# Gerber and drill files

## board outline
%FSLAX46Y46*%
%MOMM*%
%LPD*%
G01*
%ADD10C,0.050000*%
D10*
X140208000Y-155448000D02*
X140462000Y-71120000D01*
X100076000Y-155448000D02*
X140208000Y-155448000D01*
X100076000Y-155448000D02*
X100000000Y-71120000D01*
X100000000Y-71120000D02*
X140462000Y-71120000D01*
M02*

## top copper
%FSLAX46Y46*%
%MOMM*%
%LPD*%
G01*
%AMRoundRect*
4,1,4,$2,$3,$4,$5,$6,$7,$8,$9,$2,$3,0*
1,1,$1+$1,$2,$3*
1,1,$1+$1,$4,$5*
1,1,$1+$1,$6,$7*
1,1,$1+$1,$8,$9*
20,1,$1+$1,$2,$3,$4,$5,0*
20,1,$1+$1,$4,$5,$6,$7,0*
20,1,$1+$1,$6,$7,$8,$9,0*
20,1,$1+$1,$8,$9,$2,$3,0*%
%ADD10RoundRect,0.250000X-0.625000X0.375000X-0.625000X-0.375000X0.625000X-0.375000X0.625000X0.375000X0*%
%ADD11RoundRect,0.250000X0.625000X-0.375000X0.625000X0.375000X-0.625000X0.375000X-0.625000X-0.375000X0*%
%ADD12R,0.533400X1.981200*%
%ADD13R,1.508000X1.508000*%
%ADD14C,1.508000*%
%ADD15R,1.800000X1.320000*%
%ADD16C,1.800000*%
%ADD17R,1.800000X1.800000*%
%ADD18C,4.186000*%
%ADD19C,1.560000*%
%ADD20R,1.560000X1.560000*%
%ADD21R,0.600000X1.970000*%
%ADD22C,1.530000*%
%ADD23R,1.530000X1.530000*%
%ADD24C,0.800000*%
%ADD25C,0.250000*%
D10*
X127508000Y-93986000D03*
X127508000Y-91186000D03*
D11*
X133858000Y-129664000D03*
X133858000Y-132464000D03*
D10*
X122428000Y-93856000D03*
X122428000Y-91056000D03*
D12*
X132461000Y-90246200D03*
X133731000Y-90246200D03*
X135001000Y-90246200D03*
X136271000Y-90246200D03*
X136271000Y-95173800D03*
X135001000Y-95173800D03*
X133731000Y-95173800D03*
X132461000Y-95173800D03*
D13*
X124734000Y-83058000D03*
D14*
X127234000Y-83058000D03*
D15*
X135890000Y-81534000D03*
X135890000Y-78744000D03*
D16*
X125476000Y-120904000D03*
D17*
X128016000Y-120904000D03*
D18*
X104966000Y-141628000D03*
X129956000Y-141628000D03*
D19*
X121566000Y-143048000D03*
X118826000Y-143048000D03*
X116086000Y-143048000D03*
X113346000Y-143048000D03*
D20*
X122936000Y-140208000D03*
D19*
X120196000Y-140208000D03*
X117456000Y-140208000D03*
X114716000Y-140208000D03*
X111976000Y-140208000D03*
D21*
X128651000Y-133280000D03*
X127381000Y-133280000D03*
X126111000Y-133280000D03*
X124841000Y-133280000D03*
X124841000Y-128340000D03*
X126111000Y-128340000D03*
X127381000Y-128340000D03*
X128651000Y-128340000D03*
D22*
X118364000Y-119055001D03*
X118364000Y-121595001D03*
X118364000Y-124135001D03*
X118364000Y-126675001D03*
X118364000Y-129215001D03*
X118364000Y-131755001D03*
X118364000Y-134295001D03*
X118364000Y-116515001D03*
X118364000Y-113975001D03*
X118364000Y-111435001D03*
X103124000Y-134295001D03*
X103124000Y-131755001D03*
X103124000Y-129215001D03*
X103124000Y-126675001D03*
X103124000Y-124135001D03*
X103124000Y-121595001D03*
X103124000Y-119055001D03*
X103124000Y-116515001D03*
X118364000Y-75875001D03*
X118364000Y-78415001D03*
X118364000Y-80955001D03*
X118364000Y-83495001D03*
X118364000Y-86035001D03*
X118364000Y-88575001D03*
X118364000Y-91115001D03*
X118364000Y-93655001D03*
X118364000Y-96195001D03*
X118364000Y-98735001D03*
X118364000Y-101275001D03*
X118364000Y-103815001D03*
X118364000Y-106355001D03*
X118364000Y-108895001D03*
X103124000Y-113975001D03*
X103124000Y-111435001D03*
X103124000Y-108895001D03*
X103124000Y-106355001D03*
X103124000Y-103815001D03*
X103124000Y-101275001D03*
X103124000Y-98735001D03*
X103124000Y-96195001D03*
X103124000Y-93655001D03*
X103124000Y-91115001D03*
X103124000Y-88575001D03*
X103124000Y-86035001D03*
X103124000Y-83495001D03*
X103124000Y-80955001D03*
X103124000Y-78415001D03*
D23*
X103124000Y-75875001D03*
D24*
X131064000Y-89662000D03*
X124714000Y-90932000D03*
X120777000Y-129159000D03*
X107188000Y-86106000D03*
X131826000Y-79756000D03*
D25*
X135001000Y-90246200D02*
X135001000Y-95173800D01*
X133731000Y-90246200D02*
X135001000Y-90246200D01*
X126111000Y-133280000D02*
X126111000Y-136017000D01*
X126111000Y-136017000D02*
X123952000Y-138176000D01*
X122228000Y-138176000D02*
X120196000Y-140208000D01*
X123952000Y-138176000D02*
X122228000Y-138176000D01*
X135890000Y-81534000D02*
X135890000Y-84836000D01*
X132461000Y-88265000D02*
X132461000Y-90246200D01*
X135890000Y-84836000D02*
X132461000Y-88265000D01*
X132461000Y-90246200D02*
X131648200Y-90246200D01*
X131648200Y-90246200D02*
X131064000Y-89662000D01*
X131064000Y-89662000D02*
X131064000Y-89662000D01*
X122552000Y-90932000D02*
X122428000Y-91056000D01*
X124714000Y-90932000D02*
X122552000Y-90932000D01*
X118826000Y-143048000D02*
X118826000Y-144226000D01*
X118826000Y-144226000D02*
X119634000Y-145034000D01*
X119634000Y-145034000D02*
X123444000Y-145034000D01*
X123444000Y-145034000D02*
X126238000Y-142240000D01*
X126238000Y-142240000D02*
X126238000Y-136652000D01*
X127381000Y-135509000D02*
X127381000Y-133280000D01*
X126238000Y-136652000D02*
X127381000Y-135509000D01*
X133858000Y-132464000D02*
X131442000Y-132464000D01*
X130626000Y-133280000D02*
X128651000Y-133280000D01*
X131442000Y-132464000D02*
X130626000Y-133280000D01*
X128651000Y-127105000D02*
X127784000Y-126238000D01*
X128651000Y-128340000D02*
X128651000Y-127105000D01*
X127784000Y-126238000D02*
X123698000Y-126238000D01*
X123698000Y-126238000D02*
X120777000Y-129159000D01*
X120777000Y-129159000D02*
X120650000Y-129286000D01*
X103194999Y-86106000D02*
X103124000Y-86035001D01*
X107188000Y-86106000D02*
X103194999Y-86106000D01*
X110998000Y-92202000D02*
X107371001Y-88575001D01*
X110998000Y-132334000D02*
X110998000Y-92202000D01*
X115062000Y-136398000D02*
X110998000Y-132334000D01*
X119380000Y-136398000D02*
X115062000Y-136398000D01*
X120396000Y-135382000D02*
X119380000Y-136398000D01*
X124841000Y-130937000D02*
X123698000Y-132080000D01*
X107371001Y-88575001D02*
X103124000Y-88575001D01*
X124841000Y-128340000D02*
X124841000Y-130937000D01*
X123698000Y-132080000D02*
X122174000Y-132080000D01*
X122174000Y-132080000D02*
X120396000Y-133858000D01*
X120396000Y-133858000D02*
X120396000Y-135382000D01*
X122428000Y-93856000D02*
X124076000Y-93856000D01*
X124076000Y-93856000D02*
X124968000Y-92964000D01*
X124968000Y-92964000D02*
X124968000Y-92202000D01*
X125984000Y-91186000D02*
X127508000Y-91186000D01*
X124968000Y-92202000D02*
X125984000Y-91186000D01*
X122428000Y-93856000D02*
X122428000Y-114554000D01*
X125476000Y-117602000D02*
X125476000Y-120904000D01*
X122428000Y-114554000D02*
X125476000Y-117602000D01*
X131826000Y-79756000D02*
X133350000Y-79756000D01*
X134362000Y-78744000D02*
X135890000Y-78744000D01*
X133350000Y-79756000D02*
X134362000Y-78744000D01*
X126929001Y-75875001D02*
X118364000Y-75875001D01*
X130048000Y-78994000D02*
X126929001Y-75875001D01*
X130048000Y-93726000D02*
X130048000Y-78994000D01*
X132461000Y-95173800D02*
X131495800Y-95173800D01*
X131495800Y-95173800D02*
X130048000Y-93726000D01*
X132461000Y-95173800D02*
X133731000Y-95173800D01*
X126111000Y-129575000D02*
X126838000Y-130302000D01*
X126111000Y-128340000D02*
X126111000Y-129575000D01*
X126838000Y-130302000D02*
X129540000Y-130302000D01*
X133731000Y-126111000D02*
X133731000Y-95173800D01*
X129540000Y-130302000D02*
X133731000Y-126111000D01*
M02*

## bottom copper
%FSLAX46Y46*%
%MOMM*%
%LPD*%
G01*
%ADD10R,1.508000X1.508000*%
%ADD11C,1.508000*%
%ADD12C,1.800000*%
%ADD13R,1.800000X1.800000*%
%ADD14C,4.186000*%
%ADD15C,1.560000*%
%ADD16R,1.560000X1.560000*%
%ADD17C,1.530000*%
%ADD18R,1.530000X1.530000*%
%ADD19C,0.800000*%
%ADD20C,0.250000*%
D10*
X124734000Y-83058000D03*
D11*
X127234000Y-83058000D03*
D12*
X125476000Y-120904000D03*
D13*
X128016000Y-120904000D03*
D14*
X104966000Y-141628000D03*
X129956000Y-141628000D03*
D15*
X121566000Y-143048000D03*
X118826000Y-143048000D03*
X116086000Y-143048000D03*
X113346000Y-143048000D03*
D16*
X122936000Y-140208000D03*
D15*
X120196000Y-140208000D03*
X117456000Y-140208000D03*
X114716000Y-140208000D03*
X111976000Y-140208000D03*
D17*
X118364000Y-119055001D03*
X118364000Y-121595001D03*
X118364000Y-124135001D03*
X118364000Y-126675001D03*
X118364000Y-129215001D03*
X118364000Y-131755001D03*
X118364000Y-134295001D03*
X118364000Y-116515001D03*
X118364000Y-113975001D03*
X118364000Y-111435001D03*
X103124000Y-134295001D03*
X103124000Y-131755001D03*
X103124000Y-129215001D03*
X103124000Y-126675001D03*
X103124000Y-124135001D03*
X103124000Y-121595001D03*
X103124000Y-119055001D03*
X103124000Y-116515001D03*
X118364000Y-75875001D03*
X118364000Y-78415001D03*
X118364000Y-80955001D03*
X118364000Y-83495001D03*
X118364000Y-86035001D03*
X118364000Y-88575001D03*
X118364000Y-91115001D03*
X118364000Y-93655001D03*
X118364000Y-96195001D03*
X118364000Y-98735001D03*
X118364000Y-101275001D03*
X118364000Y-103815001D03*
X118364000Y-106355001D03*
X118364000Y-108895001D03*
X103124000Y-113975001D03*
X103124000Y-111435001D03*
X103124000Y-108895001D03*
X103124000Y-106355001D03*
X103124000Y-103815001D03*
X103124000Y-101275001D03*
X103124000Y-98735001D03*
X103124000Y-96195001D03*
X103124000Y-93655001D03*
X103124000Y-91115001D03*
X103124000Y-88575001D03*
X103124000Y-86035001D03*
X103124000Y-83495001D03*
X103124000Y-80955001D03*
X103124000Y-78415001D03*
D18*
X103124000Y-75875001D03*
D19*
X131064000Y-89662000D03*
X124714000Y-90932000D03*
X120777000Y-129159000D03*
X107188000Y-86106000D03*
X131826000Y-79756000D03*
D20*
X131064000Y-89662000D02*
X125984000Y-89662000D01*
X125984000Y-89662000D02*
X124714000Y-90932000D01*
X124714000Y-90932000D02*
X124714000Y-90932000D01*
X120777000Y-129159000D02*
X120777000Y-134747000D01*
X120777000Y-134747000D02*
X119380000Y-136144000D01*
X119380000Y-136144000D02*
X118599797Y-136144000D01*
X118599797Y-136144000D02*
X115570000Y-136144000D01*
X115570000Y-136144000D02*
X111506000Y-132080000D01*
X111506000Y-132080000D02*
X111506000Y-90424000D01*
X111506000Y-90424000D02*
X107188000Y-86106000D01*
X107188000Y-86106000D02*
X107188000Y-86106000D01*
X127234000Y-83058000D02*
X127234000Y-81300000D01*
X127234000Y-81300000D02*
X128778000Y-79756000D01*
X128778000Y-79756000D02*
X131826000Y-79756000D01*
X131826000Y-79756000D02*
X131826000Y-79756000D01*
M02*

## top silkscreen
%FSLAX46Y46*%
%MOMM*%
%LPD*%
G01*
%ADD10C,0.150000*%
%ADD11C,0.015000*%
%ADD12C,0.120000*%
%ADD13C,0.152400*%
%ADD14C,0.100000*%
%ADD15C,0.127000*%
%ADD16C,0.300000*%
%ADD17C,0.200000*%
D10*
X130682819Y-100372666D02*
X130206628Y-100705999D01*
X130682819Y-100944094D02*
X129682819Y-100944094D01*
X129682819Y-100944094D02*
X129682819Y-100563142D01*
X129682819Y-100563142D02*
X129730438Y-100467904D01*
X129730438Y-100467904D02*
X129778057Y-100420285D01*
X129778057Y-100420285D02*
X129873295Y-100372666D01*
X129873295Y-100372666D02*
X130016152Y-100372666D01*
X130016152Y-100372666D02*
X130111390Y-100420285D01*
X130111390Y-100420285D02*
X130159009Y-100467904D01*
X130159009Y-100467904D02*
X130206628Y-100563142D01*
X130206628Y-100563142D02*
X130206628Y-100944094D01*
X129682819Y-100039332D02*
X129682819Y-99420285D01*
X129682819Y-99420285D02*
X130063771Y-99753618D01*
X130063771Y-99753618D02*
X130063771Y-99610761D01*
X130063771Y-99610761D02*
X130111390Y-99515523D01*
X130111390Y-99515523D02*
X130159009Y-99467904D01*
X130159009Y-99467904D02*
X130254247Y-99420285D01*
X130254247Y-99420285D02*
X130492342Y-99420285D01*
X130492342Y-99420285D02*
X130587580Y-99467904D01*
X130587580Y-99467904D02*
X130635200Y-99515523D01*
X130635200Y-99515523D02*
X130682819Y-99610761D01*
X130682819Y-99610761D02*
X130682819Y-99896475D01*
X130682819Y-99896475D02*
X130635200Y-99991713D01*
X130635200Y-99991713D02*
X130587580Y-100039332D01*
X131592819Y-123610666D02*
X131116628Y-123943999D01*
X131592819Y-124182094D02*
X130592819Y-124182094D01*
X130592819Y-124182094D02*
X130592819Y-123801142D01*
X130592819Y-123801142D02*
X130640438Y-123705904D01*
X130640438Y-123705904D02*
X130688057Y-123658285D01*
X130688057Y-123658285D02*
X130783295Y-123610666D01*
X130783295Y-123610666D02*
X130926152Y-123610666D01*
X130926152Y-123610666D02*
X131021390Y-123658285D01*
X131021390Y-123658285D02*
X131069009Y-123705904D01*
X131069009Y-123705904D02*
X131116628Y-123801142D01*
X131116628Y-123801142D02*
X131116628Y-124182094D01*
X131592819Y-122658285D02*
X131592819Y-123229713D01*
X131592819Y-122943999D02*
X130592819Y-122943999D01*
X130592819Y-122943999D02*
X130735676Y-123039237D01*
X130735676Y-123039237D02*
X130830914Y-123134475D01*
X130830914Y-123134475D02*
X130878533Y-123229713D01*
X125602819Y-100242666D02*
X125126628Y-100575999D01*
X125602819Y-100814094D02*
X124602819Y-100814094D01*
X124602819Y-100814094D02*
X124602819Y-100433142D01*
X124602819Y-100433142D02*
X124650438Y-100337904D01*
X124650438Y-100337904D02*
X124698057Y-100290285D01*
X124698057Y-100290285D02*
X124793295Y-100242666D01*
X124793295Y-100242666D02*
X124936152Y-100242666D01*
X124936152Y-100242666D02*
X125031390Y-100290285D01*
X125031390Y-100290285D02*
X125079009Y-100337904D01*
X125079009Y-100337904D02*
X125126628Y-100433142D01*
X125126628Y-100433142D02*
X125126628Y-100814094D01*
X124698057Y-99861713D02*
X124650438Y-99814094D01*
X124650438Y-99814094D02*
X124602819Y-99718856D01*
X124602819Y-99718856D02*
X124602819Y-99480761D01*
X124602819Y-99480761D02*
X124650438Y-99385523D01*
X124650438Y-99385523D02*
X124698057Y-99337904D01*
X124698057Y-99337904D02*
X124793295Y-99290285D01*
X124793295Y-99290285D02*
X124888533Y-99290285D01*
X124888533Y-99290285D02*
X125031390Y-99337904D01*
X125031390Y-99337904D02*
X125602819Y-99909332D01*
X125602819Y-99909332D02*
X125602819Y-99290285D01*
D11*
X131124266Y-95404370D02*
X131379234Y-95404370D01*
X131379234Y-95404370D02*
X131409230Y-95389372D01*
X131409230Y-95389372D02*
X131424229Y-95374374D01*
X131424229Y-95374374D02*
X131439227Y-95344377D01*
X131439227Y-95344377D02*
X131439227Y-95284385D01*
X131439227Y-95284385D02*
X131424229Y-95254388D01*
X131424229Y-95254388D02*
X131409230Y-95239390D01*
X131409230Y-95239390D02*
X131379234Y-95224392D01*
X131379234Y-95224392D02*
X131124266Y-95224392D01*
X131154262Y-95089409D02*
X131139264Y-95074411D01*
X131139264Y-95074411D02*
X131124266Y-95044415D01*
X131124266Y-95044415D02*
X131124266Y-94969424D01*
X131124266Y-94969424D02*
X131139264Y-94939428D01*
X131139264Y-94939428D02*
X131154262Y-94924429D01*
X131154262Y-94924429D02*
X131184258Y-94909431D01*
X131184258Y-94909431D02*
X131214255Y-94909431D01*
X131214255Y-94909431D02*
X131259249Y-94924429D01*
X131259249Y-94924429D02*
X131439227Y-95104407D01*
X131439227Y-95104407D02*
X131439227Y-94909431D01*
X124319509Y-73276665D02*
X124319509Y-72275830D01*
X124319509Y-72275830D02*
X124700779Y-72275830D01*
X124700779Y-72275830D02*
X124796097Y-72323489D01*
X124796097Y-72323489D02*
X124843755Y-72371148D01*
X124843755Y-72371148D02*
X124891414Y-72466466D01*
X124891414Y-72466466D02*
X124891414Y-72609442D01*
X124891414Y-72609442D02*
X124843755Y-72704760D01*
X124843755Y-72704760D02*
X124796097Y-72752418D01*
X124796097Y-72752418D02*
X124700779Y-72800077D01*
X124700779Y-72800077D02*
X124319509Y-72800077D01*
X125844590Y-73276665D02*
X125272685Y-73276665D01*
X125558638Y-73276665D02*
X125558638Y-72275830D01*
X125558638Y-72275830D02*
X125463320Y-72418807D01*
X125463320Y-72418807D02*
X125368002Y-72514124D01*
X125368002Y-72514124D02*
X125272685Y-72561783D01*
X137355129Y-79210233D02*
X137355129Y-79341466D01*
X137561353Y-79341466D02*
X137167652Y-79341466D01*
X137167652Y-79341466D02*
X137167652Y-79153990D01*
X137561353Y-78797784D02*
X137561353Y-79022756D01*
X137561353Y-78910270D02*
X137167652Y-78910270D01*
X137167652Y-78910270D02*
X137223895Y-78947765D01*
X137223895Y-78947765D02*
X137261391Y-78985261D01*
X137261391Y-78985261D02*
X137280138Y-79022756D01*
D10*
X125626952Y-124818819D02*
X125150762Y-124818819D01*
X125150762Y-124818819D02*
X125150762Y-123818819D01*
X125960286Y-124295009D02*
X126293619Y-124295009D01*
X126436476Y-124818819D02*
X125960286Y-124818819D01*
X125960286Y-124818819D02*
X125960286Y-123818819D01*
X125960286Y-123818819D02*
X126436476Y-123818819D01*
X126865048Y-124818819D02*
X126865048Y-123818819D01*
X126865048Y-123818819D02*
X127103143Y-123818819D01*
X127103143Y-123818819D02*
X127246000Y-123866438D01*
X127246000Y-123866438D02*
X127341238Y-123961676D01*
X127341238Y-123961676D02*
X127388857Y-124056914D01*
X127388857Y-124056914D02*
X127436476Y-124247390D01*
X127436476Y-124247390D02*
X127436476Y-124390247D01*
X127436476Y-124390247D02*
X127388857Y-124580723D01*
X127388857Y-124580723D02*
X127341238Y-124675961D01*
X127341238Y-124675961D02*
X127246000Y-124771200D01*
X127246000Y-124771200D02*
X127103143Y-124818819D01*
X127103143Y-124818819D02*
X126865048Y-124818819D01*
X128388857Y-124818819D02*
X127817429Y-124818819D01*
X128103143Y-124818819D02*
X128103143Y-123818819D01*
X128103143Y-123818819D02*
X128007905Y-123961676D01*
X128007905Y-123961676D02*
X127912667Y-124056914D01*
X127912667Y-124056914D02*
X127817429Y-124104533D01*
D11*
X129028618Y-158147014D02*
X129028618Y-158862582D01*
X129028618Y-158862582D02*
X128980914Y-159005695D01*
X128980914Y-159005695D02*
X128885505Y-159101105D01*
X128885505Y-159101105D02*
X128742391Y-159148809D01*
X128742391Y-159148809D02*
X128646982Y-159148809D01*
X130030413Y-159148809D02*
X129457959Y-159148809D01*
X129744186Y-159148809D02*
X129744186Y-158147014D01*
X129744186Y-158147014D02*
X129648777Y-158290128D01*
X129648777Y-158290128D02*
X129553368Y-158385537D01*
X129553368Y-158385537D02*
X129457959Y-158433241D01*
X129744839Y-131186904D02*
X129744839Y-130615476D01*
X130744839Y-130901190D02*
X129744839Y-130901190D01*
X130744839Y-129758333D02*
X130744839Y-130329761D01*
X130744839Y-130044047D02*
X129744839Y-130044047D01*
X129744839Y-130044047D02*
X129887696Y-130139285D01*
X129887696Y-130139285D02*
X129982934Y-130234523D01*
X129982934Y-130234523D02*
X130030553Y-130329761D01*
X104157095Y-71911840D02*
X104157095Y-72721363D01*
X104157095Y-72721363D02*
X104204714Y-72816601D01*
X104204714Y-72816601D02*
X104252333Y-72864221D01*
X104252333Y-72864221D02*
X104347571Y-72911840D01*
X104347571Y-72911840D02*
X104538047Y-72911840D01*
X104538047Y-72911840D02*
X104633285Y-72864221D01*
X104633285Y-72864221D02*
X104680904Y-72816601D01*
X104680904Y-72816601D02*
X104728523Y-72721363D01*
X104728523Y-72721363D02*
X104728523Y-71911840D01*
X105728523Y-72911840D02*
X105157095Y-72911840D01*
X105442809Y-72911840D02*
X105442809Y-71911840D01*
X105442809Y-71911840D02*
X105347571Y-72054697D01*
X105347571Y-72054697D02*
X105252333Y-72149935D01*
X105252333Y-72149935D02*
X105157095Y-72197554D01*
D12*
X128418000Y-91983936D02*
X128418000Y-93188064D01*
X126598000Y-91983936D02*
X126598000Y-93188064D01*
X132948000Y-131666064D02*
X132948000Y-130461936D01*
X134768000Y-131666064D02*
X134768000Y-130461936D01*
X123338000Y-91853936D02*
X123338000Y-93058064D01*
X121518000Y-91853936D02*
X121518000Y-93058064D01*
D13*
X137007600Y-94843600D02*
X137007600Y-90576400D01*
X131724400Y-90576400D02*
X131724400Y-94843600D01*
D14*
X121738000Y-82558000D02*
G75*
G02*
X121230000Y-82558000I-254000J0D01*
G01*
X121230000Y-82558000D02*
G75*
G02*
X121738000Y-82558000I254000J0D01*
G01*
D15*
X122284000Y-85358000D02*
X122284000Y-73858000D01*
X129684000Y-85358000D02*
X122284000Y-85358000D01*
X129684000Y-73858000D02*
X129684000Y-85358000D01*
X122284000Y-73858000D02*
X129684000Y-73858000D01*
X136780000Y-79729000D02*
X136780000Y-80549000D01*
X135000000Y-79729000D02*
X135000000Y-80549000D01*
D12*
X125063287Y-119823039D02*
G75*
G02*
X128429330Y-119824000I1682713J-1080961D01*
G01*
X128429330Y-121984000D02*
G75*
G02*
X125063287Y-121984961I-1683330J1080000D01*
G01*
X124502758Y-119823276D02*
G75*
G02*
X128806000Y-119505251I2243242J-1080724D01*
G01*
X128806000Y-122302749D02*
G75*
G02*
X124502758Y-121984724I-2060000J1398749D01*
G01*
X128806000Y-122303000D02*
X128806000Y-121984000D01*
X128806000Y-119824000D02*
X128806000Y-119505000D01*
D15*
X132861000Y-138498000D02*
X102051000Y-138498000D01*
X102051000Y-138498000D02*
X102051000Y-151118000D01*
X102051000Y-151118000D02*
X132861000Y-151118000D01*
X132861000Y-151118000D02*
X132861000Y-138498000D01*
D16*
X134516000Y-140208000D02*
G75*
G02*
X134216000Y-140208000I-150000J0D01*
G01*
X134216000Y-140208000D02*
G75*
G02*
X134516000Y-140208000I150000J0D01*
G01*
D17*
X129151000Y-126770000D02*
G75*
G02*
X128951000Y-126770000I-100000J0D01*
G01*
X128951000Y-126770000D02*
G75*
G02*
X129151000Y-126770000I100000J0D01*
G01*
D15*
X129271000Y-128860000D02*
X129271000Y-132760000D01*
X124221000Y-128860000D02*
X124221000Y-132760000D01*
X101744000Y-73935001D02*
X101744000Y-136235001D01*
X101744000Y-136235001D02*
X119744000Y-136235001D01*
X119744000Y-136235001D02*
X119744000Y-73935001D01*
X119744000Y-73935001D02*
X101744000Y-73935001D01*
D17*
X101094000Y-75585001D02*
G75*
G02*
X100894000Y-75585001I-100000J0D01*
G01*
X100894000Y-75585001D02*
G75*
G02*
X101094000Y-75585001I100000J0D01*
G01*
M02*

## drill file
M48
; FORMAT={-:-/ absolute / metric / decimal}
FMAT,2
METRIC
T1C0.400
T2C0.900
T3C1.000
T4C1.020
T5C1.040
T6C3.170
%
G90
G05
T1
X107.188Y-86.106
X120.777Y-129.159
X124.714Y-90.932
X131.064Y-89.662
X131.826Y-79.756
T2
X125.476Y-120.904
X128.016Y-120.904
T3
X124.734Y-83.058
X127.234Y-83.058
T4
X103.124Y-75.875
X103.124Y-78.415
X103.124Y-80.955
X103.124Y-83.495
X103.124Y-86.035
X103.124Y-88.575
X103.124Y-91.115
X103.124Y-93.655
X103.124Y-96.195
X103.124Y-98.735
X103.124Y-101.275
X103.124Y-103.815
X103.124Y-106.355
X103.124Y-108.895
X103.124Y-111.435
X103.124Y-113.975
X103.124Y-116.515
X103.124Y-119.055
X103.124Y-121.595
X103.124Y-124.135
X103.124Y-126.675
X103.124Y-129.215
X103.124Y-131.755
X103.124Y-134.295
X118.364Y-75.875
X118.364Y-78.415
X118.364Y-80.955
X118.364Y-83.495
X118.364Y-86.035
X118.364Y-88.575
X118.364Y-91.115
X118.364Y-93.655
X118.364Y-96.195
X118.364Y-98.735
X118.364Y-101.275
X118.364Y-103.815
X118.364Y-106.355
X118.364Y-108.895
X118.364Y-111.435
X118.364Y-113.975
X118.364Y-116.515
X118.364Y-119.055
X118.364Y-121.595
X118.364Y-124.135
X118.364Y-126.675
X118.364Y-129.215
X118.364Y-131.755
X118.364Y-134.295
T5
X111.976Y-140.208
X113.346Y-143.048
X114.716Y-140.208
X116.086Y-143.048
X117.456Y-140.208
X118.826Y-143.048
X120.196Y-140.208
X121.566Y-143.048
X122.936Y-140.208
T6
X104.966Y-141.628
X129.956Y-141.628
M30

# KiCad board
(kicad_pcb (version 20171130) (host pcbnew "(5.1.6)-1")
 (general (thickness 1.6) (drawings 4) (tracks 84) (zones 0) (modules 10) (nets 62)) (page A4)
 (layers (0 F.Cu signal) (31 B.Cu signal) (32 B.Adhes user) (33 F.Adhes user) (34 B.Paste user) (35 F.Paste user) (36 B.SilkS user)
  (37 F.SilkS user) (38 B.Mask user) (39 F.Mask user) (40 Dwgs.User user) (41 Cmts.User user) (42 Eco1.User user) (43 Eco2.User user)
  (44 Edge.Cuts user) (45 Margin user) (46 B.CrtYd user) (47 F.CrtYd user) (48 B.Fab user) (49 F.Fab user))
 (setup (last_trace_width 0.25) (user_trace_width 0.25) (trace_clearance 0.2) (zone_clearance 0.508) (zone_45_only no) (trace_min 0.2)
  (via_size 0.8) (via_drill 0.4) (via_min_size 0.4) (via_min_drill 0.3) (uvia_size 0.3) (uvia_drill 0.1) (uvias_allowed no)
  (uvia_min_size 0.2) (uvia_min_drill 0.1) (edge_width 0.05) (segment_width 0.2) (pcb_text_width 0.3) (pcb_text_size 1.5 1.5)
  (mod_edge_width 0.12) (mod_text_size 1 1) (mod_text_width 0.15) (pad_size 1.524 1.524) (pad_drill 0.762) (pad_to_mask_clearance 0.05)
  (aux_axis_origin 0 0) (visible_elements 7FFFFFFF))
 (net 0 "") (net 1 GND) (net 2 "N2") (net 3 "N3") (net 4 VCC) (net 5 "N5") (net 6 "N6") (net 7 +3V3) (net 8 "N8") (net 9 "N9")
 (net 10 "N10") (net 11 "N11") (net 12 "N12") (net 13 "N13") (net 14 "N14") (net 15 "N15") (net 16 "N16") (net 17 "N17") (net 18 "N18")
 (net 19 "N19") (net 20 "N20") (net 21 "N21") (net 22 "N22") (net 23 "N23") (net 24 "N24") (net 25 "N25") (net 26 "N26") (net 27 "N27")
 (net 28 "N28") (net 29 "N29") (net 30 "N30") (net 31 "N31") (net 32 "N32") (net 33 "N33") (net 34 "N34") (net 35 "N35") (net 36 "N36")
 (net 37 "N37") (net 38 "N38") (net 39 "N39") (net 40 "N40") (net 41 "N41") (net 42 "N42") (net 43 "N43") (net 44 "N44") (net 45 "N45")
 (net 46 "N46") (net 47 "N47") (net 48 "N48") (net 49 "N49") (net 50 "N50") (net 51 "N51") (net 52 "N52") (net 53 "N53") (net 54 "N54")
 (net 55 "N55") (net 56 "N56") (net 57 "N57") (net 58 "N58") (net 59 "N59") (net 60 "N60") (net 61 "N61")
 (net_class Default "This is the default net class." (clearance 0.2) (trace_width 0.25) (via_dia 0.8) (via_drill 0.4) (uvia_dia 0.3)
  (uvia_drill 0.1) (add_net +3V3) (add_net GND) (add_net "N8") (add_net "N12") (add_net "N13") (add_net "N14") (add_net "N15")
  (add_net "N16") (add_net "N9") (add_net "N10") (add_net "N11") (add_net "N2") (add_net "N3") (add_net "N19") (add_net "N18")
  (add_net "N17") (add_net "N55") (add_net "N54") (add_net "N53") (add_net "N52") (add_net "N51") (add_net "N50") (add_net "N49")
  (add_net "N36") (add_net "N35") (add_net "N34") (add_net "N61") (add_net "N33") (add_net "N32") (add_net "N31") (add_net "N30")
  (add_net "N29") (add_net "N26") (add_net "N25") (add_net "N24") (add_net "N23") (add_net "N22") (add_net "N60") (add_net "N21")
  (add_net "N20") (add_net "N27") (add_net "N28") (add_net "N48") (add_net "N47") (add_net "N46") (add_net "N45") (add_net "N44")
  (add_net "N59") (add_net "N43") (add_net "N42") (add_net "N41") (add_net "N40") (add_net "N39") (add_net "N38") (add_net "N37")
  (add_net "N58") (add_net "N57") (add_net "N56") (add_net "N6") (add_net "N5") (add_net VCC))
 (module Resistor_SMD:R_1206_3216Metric (layer F.Cu) (at 127.508 92.586 270)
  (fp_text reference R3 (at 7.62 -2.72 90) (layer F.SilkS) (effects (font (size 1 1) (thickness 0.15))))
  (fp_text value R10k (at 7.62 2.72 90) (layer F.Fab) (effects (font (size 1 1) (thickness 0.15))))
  (fp_line (start -0.602064 -0.91) (end 0.602064 -0.91) (layer F.SilkS) (width 0.12))
  (fp_line (start -0.602064 0.91) (end 0.602064 0.91) (layer F.SilkS) (width 0.12))
  (pad 2 smd roundrect (at 1.4 0 270) (size 1.25 1.75) (layers F.Cu F.Paste F.Mask) (roundrect_rratio 0.2) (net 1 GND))
  (pad 1 smd roundrect (at -1.4 0 270) (size 1.25 1.75) (layers F.Cu F.Paste F.Mask) (roundrect_rratio 0.2) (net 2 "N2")))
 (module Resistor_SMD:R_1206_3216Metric (layer F.Cu) (at 133.858 131.064 90)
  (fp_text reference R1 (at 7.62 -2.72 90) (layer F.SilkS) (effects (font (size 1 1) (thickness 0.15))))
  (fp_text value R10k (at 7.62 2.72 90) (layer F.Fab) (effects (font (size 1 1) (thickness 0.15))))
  (fp_line (start -0.602064 -0.91) (end 0.602064 -0.91) (layer F.SilkS) (width 0.12))
  (fp_line (start -0.602064 0.91) (end 0.602064 0.91) (layer F.SilkS) (width 0.12))
  (pad 2 smd roundrect (at 1.4 0 90) (size 1.25 1.75) (layers F.Cu F.Paste F.Mask) (roundrect_rratio 0.2) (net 1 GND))
  (pad 1 smd roundrect (at -1.4 0 90) (size 1.25 1.75) (layers F.Cu F.Paste F.Mask) (roundrect_rratio 0.2) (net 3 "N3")))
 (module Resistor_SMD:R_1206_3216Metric (layer F.Cu) (at 122.428 92.456 270)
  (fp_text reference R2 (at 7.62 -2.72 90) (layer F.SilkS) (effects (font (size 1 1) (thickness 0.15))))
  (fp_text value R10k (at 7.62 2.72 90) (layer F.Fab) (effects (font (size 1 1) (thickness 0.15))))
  (fp_line (start -0.602064 -0.91) (end 0.602064 -0.91) (layer F.SilkS) (width 0.12))
  (fp_line (start -0.602064 0.91) (end 0.602064 0.91) (layer F.SilkS) (width 0.12))
  (pad 2 smd roundrect (at 1.4 0 270) (size 1.25 1.75) (layers F.Cu F.Paste F.Mask) (roundrect_rratio 0.2) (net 2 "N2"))
  (pad 1 smd roundrect (at -1.4 0 270) (size 1.25 1.75) (layers F.Cu F.Paste F.Mask) (roundrect_rratio 0.2) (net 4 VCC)))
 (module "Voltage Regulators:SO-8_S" (layer F.Cu) (at 134.366 92.71 90)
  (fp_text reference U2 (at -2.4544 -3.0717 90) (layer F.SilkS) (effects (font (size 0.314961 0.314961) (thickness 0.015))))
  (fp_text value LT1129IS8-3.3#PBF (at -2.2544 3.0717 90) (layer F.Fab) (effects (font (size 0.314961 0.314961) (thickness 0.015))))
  (fp_line (start -2.1336 2.6416) (end 2.1336 2.6416) (layer F.SilkS) (width 0.1524))
  (fp_line (start 2.1336 -2.6416) (end -2.1336 -2.6416) (layer F.SilkS) (width 0.1524))
  (pad 8 smd rect (at 2.4638 -1.905 90) (size 1.9812 0.5334) (layers F.Cu F.Paste F.Mask) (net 4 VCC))
  (pad 7 smd rect (at 2.4638 -0.635 90) (size 1.9812 0.5334) (layers F.Cu F.Paste F.Mask) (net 1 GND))
  (pad 6 smd rect (at 2.4638 0.635 90) (size 1.9812 0.5334) (layers F.Cu F.Paste F.Mask) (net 1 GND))
  (pad 5 smd rect (at 2.4638 1.905 90) (size 1.9812 0.5334) (layers F.Cu F.Paste F.Mask) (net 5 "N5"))
  (pad 4 smd rect (at -2.4638 1.905 90) (size 1.9812 0.5334) (layers F.Cu F.Paste F.Mask) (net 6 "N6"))
  (pad 3 smd rect (at -2.4638 0.635 90) (size 1.9812 0.5334) (layers F.Cu F.Paste F.Mask) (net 1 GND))
  (pad 2 smd rect (at -2.4638 -0.635 90) (size 1.9812 0.5334) (layers F.Cu F.Paste F.Mask) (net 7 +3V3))
  (pad 1 smd rect (at -2.4638 -1.905 90) (size 1.9812 0.5334) (layers F.Cu F.Paste F.Mask) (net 7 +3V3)))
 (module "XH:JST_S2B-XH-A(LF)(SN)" (layer F.Cu) (at 125.984 83.058)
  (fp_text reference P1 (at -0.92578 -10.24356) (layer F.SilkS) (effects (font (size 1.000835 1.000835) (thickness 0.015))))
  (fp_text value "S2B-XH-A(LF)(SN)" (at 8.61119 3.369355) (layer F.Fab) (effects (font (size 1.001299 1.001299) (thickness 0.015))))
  (fp_circle (center -4.5 -0.5) (end -4.246 -0.5) (layer F.SilkS) (width 0.1))
  (fp_line (start -3.7 2.3) (end -3.7 -9.2) (layer F.SilkS) (width 0.127))
  (fp_line (start 3.7 2.3) (end -3.7 2.3) (layer F.SilkS) (width 0.127))
  (fp_line (start 3.7 -9.2) (end 3.7 2.3) (layer F.SilkS) (width 0.127))
  (fp_line (start -3.7 -9.2) (end 3.7 -9.2) (layer F.SilkS) (width 0.127))
  (pad 1 thru_hole rect (at -1.25 0) (size 1.508 1.508) (drill 1) (layers *.Cu *.Mask) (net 1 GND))
  (pad 2 thru_hole circle (at 1.25 0) (size 1.508 1.508) (drill 1) (layers *.Cu *.Mask) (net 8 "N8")))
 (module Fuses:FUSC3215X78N (layer F.Cu) (at 135.89 80.139 270)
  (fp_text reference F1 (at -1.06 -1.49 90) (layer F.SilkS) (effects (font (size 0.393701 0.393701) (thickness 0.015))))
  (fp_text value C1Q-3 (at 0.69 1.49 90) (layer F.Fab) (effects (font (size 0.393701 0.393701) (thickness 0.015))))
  (fp_line (start -0.41 -0.89) (end 0.41 -0.89) (layer F.SilkS) (width 0.127))
  (fp_line (start -0.41 0.89) (end 0.41 0.89) (layer F.SilkS) (width 0.127))
  (pad 2 smd rect (at 1.395 0 270) (size 1.32 1.8) (layers F.Cu F.Paste F.Mask) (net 4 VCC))
  (pad 1 smd rect (at -1.395 0 270) (size 1.32 1.8) (layers F.Cu F.Paste F.Mask) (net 8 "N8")))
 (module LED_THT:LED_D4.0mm (layer F.Cu) (at 128.016 120.904 180)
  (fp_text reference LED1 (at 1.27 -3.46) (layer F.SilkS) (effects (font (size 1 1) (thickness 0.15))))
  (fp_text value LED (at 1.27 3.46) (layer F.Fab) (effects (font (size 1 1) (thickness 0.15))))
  (fp_arc (start 1.27 0) (end -0.41333 1.08) (angle -114.6) (layer F.SilkS) (width 0.12))
  (fp_arc (start 1.27 0) (end -0.41333 -1.08) (angle 114.6) (layer F.SilkS) (width 0.12))
  (fp_arc (start 1.27 0) (end -0.79 1.398749) (angle -120.1) (layer F.SilkS) (width 0.12))
  (fp_arc (start 1.27 0) (end -0.79 -1.398749) (angle 120.1) (layer F.SilkS) (width 0.12))
  (fp_line (start -0.79 -1.399) (end -0.79 -1.08) (layer F.SilkS) (width 0.12))
  (fp_line (start -0.79 1.08) (end -0.79 1.399) (layer F.SilkS) (width 0.12))
  (pad 2 thru_hole circle (at 2.54 0 180) (size 1.8 1.8) (drill 0.9) (layers *.Cu *.Mask) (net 2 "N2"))
  (pad 1 thru_hole rect (at 0 0 180) (size 1.8 1.8) (drill 0.9) (layers *.Cu *.Mask) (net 1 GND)))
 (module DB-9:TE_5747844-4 (layer F.Cu) (at 122.936 140.208 180)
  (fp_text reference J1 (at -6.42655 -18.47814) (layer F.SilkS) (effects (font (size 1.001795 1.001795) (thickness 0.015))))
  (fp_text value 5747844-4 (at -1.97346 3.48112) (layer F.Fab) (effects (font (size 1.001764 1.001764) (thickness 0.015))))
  (fp_line (start -9.925 1.71) (end 20.885 1.71) (layer F.SilkS) (width 0.127))
  (fp_line (start 20.885 1.71) (end 20.885 -10.91) (layer F.SilkS) (width 0.127))
  (fp_line (start 20.885 -10.91) (end -9.925 -10.91) (layer F.SilkS) (width 0.127))
  (fp_line (start -9.925 -10.91) (end -9.925 1.71) (layer F.SilkS) (width 0.127))
  (fp_circle (center -11.43 0) (end -11.28 0) (layer F.SilkS) (width 0.3))
  (pad SH2 thru_hole circle (at 17.97 -1.42 180) (size 4.186 4.186) (drill 3.17) (layers *.Cu *.Mask) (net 1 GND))
  (pad SH1 thru_hole circle (at -7.02 -1.42 180) (size 4.186 4.186) (drill 3.17) (layers *.Cu *.Mask) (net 1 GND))
  (pad 6 thru_hole circle (at 1.37 -2.84 180) (size 1.56 1.56) (drill 1.04) (layers *.Cu *.Mask) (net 1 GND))
  (pad 7 thru_hole circle (at 4.11 -2.84 180) (size 1.56 1.56) (drill 1.04) (layers *.Cu *.Mask) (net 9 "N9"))
  (pad 8 thru_hole circle (at 6.85 -2.84 180) (size 1.56 1.56) (drill 1.04) (layers *.Cu *.Mask) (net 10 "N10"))
  (pad 9 thru_hole circle (at 9.59 -2.84 180) (size 1.56 1.56) (drill 1.04) (layers *.Cu *.Mask) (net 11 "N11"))
  (pad 1 thru_hole rect (at 0 0 180) (size 1.56 1.56) (drill 1.04) (layers *.Cu *.Mask) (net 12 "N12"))
  (pad 2 thru_hole circle (at 2.74 0 180) (size 1.56 1.56) (drill 1.04) (layers *.Cu *.Mask) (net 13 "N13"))
  (pad 3 thru_hole circle (at 5.48 0 180) (size 1.56 1.56) (drill 1.04) (layers *.Cu *.Mask) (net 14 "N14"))
  (pad 4 thru_hole circle (at 8.22 0 180) (size 1.56 1.56) (drill 1.04) (layers *.Cu *.Mask) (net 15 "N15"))
  (pad 5 thru_hole circle (at 10.96 0 180) (size 1.56 1.56) (drill 1.04) (layers *.Cu *.Mask) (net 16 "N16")))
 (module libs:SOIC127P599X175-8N (layer F.Cu) (at 126.746 130.81 270)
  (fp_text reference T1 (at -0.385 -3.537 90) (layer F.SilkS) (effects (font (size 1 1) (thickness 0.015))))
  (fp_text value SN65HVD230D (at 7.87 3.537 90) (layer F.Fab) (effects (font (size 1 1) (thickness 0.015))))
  (fp_circle (center -4.04 -2.305) (end -3.94 -2.305) (layer F.SilkS) (width 0.2))
  (fp_line (start -1.95 -2.525) (end 1.95 -2.525) (layer F.SilkS) (width 0.127))
  (fp_line (start -1.95 2.525) (end 1.95 2.525) (layer F.SilkS) (width 0.127))
  (pad 8 smd rect (at 2.47 -1.905 270) (size 1.97 0.6) (layers F.Cu F.Paste F.Mask) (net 3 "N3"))
  (pad 7 smd rect (at 2.47 -0.635 270) (size 1.97 0.6) (layers F.Cu F.Paste F.Mask) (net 9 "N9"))
  (pad 6 smd rect (at 2.47 0.635 270) (size 1.97 0.6) (layers F.Cu F.Paste F.Mask) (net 13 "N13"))
  (pad 5 smd rect (at 2.47 1.905 270) (size 1.97 0.6) (layers F.Cu F.Paste F.Mask) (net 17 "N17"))
  (pad 4 smd rect (at -2.47 1.905 270) (size 1.97 0.6) (layers F.Cu F.Paste F.Mask) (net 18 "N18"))
  (pad 3 smd rect (at -2.47 0.635 270) (size 1.97 0.6) (layers F.Cu F.Paste F.Mask) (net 7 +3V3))
  (pad 2 smd rect (at -2.47 -0.635 270) (size 1.97 0.6) (layers F.Cu F.Paste F.Mask) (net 1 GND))
  (pad 1 smd rect (at -2.47 -1.905 270) (size 1.97 0.6) (layers F.Cu F.Paste F.Mask) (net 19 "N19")))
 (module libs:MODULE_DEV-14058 (layer F.Cu) (at 110.744 105.085001)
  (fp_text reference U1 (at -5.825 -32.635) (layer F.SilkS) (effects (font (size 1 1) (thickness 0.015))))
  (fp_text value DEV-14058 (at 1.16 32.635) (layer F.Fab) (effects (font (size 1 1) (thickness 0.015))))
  (fp_line (start -9 -31.15) (end -9 31.15) (layer F.SilkS) (width 0.127))
  (fp_line (start -9 31.15) (end 9 31.15) (layer F.SilkS) (width 0.127))
  (fp_line (start 9 31.15) (end 9 -31.15) (layer F.SilkS) (width 0.127))
  (fp_line (start 9 -31.15) (end -9 -31.15) (layer F.SilkS) (width 0.127))
  (fp_circle (center -9.75 -29.5) (end -9.65 -29.5) (layer F.SilkS) (width 0.2))
  (pad 31 thru_hole circle (at 7.62 13.97) (size 1.53 1.53) (drill 1.02) (layers *.Cu *.Mask) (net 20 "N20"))
  (pad 30 thru_hole circle (at 7.62 16.51) (size 1.53 1.53) (drill 1.02) (layers *.Cu *.Mask) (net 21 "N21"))
  (pad 29 thru_hole circle (at 7.62 19.05) (size 1.53 1.53) (drill 1.02) (layers *.Cu *.Mask) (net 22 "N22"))
  (pad 28 thru_hole circle (at 7.62 21.59) (size 1.53 1.53) (drill 1.02) (layers *.Cu *.Mask) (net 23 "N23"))
  (pad 27 thru_hole circle (at 7.62 24.13) (size 1.53 1.53) (drill 1.02) (layers *.Cu *.Mask) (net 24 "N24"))
  (pad 26 thru_hole circle (at 7.62 26.67) (size 1.53 1.53) (drill 1.02) (layers *.Cu *.Mask) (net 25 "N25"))
  (pad 25 thru_hole circle (at 7.62 29.21) (size 1.53 1.53) (drill 1.02) (layers *.Cu *.Mask) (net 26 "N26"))
  (pad 32 thru_hole circle (at 7.62 11.43) (size 1.53 1.53) (drill 1.02) (layers *.Cu *.Mask) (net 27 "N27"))
  (pad 33 thru_hole circle (at 7.62 8.89) (size 1.53 1.53) (drill 1.02) (layers *.Cu *.Mask) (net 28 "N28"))
  (pad 34 thru_hole circle (at 7.62 6.35) (size 1.53 1.53) (drill 1.02) (layers *.Cu *.Mask) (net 1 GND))
  (pad 24 thru_hole circle (at -7.62 29.21) (size 1.53 1.53) (drill 1.02) (layers *.Cu *.Mask) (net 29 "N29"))
  (pad 23 thru_hole circle (at -7.62 26.67) (size 1.53 1.53) (drill 1.02) (layers *.Cu *.Mask) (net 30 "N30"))
  (pad 22 thru_hole circle (at -7.62 24.13) (size 1.53 1.53) (drill 1.02) (layers *.Cu *.Mask) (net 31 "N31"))
  (pad 21 thru_hole circle (at -7.62 21.59) (size 1.53 1.53) (drill 1.02) (layers *.Cu *.Mask) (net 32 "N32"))
  (pad 20 thru_hole circle (at -7.62 19.05) (size 1.53 1.53) (drill 1.02) (layers *.Cu *.Mask) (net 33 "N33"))
  (pad 19 thru_hole circle (at -7.62 16.51) (size 1.53 1.53) (drill 1.02) (layers *.Cu *.Mask) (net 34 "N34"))
  (pad 18 thru_hole circle (at -7.62 13.97) (size 1.53 1.53) (drill 1.02) (layers *.Cu *.Mask) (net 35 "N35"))
  (pad 17 thru_hole circle (at -7.62 11.43) (size 1.53 1.53) (drill 1.02) (layers *.Cu *.Mask) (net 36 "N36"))
  (pad 48 thru_hole circle (at 7.62 -29.21) (size 1.53 1.53) (drill 1.02) (layers *.Cu *.Mask) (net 7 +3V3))
  (pad 47 thru_hole circle (at 7.62 -26.67) (size 1.53 1.53) (drill 1.02) (layers *.Cu *.Mask) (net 1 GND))
  (pad 46 thru_hole circle (at 7.62 -24.13) (size 1.53 1.53) (drill 1.02) (layers *.Cu *.Mask) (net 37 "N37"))
  (pad 45 thru_hole circle (at 7.62 -21.59) (size 1.53 1.53) (drill 1.02) (layers *.Cu *.Mask) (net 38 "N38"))
  (pad 44 thru_hole circle (at 7.62 -19.05) (size 1.53 1.53) (drill 1.02) (layers *.Cu *.Mask) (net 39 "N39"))
  (pad 43 thru_hole circle (at 7.62 -16.51) (size 1.53 1.53) (drill 1.02) (layers *.Cu *.Mask) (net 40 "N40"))
  (pad 42 thru_hole circle (at 7.62 -13.97) (size 1.53 1.53) (drill 1.02) (layers *.Cu *.Mask) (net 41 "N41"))
  (pad 41 thru_hole circle (at 7.62 -11.43) (size 1.53 1.53) (drill 1.02) (layers *.Cu *.Mask) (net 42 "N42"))
  (pad 40 thru_hole circle (at 7.62 -8.89) (size 1.53 1.53) (drill 1.02) (layers *.Cu *.Mask) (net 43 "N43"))
  (pad 39 thru_hole circle (at 7.62 -6.35) (size 1.53 1.53) (drill 1.02) (layers *.Cu *.Mask) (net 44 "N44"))
  (pad 38 thru_hole circle (at 7.62 -3.81) (size 1.53 1.53) (drill 1.02) (layers *.Cu *.Mask) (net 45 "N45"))
  (pad 37 thru_hole circle (at 7.62 -1.27) (size 1.53 1.53) (drill 1.02) (layers *.Cu *.Mask) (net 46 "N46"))
  (pad 36 thru_hole circle (at 7.62 1.27) (size 1.53 1.53) (drill 1.02) (layers *.Cu *.Mask) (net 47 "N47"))
  (pad 35 thru_hole circle (at 7.62 3.81) (size 1.53 1.53) (drill 1.02) (layers *.Cu *.Mask) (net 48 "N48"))
  (pad 16 thru_hole circle (at -7.62 8.89) (size 1.53 1.53) (drill 1.02) (layers *.Cu *.Mask) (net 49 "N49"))
  (pad 15 thru_hole circle (at -7.62 6.35) (size 1.53 1.53) (drill 1.02) (layers *.Cu *.Mask) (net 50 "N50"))
  (pad 14 thru_hole circle (at -7.62 3.81) (size 1.53 1.53) (drill 1.02) (layers *.Cu *.Mask) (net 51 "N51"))
  (pad 13 thru_hole circle (at -7.62 1.27) (size 1.53 1.53) (drill 1.02) (layers *.Cu *.Mask) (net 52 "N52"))
  (pad 12 thru_hole circle (at -7.62 -1.27) (size 1.53 1.53) (drill 1.02) (layers *.Cu *.Mask) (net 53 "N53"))
  (pad 11 thru_hole circle (at -7.62 -3.81) (size 1.53 1.53) (drill 1.02) (layers *.Cu *.Mask) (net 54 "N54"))
  (pad 10 thru_hole circle (at -7.62 -6.35) (size 1.53 1.53) (drill 1.02) (layers *.Cu *.Mask) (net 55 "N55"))
  (pad 9 thru_hole circle (at -7.62 -8.89) (size 1.53 1.53) (drill 1.02) (layers *.Cu *.Mask) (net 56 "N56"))
  (pad 8 thru_hole circle (at -7.62 -11.43) (size 1.53 1.53) (drill 1.02) (layers *.Cu *.Mask) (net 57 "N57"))
  (pad 7 thru_hole circle (at -7.62 -13.97) (size 1.53 1.53) (drill 1.02) (layers *.Cu *.Mask) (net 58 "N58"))
  (pad 6 thru_hole circle (at -7.62 -16.51) (size 1.53 1.53) (drill 1.02) (layers *.Cu *.Mask) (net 18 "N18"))
  (pad 5 thru_hole circle (at -7.62 -19.05) (size 1.53 1.53) (drill 1.02) (layers *.Cu *.Mask) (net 19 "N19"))
  (pad 4 thru_hole circle (at -7.62 -21.59) (size 1.53 1.53) (drill 1.02) (layers *.Cu *.Mask) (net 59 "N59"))
  (pad 3 thru_hole circle (at -7.62 -24.13) (size 1.53 1.53) (drill 1.02) (layers *.Cu *.Mask) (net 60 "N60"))
  (pad 2 thru_hole circle (at -7.62 -26.67) (size 1.53 1.53) (drill 1.02) (layers *.Cu *.Mask) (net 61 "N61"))
  (pad 1 thru_hole rect (at -7.62 -29.21) (size 1.53 1.53) (drill 1.02) (layers *.Cu *.Mask) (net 1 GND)))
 (gr_line (start 140.208 155.448) (end 140.462 71.12) (layer Edge.Cuts) (width 0.05))
 (gr_line (start 100.076 155.448) (end 140.208 155.448) (layer Edge.Cuts) (width 0.05))
 (gr_line (start 100.076 155.448) (end 100 71.12) (layer Edge.Cuts) (width 0.05))
 (gr_line (start 100 71.12) (end 140.462 71.12) (layer Edge.Cuts) (width 0.05))
 (segment (start 135.001 90.2462) (end 135.001 95.1738) (width 0.25) (layer F.Cu) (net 1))
 (segment (start 133.731 90.2462) (end 135.001 90.2462) (width 0.25) (layer F.Cu) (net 1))
 (segment (start 126.111 133.28) (end 126.111 136.017) (width 0.25) (layer F.Cu) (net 13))
 (segment (start 126.111 136.017) (end 123.952 138.176) (width 0.25) (layer F.Cu) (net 13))
 (segment (start 122.228 138.176) (end 120.196 140.208) (width 0.25) (layer F.Cu) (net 13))
 (segment (start 123.952 138.176) (end 122.228 138.176) (width 0.25) (layer F.Cu) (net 13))
 (segment (start 135.89 81.534) (end 135.89 84.836) (width 0.25) (layer F.Cu) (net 4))
 (segment (start 132.461 88.265) (end 132.461 90.2462) (width 0.25) (layer F.Cu) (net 4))
 (segment (start 135.89 84.836) (end 132.461 88.265) (width 0.25) (layer F.Cu) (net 4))
 (segment (start 132.461 90.2462) (end 131.6482 90.2462) (width 0.25) (layer F.Cu) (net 4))
 (segment (start 131.6482 90.2462) (end 131.064 89.662) (width 0.25) (layer F.Cu) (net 4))
 (segment (start 131.064 89.662) (end 131.064 89.662) (width 0.25) (layer F.Cu) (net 4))
 (via (at 131.064 89.662) (size 0.8) (drill 0.4) (layers F.Cu B.Cu) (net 4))
 (segment (start 131.064 89.662) (end 125.984 89.662) (width 0.25) (layer B.Cu) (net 4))
 (segment (start 125.984 89.662) (end 124.714 90.932) (width 0.25) (layer B.Cu) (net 4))
 (segment (start 124.714 90.932) (end 124.714 90.932) (width 0.25) (layer B.Cu) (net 4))
 (via (at 124.714 90.932) (size 0.8) (drill 0.4) (layers F.Cu B.Cu) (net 4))
 (segment (start 122.552 90.932) (end 122.428 91.056) (width 0.25) (layer F.Cu) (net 4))
 (segment (start 124.714 90.932) (end 122.552 90.932) (width 0.25) (layer F.Cu) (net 4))
 (segment (start 118.826 143.048) (end 118.826 144.226) (width 0.25) (layer F.Cu) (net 9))
 (segment (start 118.826 144.226) (end 119.634 145.034) (width 0.25) (layer F.Cu) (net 9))
 (segment (start 119.634 145.034) (end 123.444 145.034) (width 0.25) (layer F.Cu) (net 9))
 (segment (start 123.444 145.034) (end 126.238 142.24) (width 0.25) (layer F.Cu) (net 9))
 (segment (start 126.238 142.24) (end 126.238 136.652) (width 0.25) (layer F.Cu) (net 9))
 (segment (start 127.381 135.509) (end 127.381 133.28) (width 0.25) (layer F.Cu) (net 9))
 (segment (start 126.238 136.652) (end 127.381 135.509) (width 0.25) (layer F.Cu) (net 9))
 (segment (start 133.858 132.464) (end 131.442 132.464) (width 0.25) (layer F.Cu) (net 3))
 (segment (start 130.626 133.28) (end 128.651 133.28) (width 0.25) (layer F.Cu) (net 3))
 (segment (start 131.442 132.464) (end 130.626 133.28) (width 0.25) (layer F.Cu) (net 3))
 (segment (start 128.651 127.105) (end 127.784 126.238) (width 0.25) (layer F.Cu) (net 19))
 (segment (start 128.651 128.34) (end 128.651 127.105) (width 0.25) (layer F.Cu) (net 19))
 (segment (start 127.784 126.238) (end 123.698 126.238) (width 0.25) (layer F.Cu) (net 19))
 (segment (start 123.698 126.238) (end 120.777 129.159) (width 0.25) (layer F.Cu) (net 19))
 (segment (start 120.777 129.159) (end 120.65 129.286) (width 0.25) (layer F.Cu) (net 19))
 (via (at 120.777 129.159) (size 0.8) (drill 0.4) (layers F.Cu B.Cu) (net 19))
 (segment (start 120.777 129.159) (end 120.777 134.747) (width 0.25) (layer B.Cu) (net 19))
 (segment (start 120.777 134.747) (end 119.38 136.144) (width 0.25) (layer B.Cu) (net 19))
 (segment (start 119.38 136.144) (end 118.599797 136.144) (width 0.25) (layer B.Cu) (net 19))
 (segment (start 118.599797 136.144) (end 115.57 136.144) (width 0.25) (layer B.Cu) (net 19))
 (segment (start 115.57 136.144) (end 111.506 132.08) (width 0.25) (layer B.Cu) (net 19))
 (segment (start 111.506 132.08) (end 111.506 90.424) (width 0.25) (layer B.Cu) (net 19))
 (segment (start 111.506 90.424) (end 107.188 86.106) (width 0.25) (layer B.Cu) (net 19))
 (segment (start 107.188 86.106) (end 107.188 86.106) (width 0.25) (layer B.Cu) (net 19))
 (via (at 107.188 86.106) (size 0.8) (drill 0.4) (layers F.Cu B.Cu) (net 19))
 (segment (start 103.194999 86.106) (end 103.124 86.035001) (width 0.25) (layer F.Cu) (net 19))
 (segment (start 107.188 86.106) (end 103.194999 86.106) (width 0.25) (layer F.Cu) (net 19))
 (segment (start 110.998 92.202) (end 107.371001 88.575001) (width 0.25) (layer F.Cu) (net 18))
 (segment (start 110.998 132.334) (end 110.998 92.202) (width 0.25) (layer F.Cu) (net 18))
 (segment (start 115.062 136.398) (end 110.998 132.334) (width 0.25) (layer F.Cu) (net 18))
 (segment (start 119.38 136.398) (end 115.062 136.398) (width 0.25) (layer F.Cu) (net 18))
 (segment (start 120.396 135.382) (end 119.38 136.398) (width 0.25) (layer F.Cu) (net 18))
 (segment (start 124.841 130.937) (end 123.698 132.08) (width 0.25) (layer F.Cu) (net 18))
 (segment (start 107.371001 88.575001) (end 103.124 88.575001) (width 0.25) (layer F.Cu) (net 18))
 (segment (start 124.841 128.34) (end 124.841 130.937) (width 0.25) (layer F.Cu) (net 18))
 (segment (start 123.698 132.08) (end 122.174 132.08) (width 0.25) (layer F.Cu) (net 18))
 (segment (start 122.174 132.08) (end 120.396 133.858) (width 0.25) (layer F.Cu) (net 18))
 (segment (start 120.396 133.858) (end 120.396 135.382) (width 0.25) (layer F.Cu) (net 18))
 (segment (start 122.428 93.856) (end 124.076 93.856) (width 0.25) (layer F.Cu) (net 2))
 (segment (start 124.076 93.856) (end 124.968 92.964) (width 0.25) (layer F.Cu) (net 2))
 (segment (start 124.968 92.964) (end 124.968 92.202) (width 0.25) (layer F.Cu) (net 2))
 (segment (start 125.984 91.186) (end 127.508 91.186) (width 0.25) (layer F.Cu) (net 2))
 (segment (start 124.968 92.202) (end 125.984 91.186) (width 0.25) (layer F.Cu) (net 2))
 (segment (start 122.428 93.856) (end 122.428 114.554) (width 0.25) (layer F.Cu) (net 2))
 (segment (start 125.476 117.602) (end 125.476 120.904) (width 0.25) (layer F.Cu) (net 2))
 (segment (start 122.428 114.554) (end 125.476 117.602) (width 0.25) (layer F.Cu) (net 2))
 (segment (start 127.234 83.058) (end 127.234 81.3) (width 0.25) (layer B.Cu) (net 8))
 (segment (start 127.234 81.3) (end 128.778 79.756) (width 0.25) (layer B.Cu) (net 8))
 (segment (start 128.778 79.756) (end 131.826 79.756) (width 0.25) (layer B.Cu) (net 8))
 (segment (start 131.826 79.756) (end 131.826 79.756) (width 0.25) (layer B.Cu) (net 8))
 (via (at 131.826 79.756) (size 0.8) (drill 0.4) (layers F.Cu B.Cu) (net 8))
 (segment (start 131.826 79.756) (end 133.35 79.756) (width 0.25) (layer F.Cu) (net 8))
 (segment (start 134.362 78.744) (end 135.89 78.744) (width 0.25) (layer F.Cu) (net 8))
 (segment (start 133.35 79.756) (end 134.362 78.744) (width 0.25) (layer F.Cu) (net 8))
 (segment (start 126.929001 75.875001) (end 118.364 75.875001) (width 0.25) (layer F.Cu) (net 7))
 (segment (start 130.048 78.994) (end 126.929001 75.875001) (width 0.25) (layer F.Cu) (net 7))
 (segment (start 130.048 93.726) (end 130.048 78.994) (width 0.25) (layer F.Cu) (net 7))
 (segment (start 132.461 95.1738) (end 131.4958 95.1738) (width 0.25) (layer F.Cu) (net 7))
 (segment (start 131.4958 95.1738) (end 130.048 93.726) (width 0.25) (layer F.Cu) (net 7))
 (segment (start 132.461 95.1738) (end 133.731 95.1738) (width 0.25) (layer F.Cu) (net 7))
 (segment (start 126.111 129.575) (end 126.838 130.302) (width 0.25) (layer F.Cu) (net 7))
 (segment (start 126.111 128.34) (end 126.111 129.575) (width 0.25) (layer F.Cu) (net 7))
 (segment (start 126.838 130.302) (end 129.54 130.302) (width 0.25) (layer F.Cu) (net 7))
 (segment (start 133.731 126.111) (end 133.731 95.1738) (width 0.25) (layer F.Cu) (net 7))
 (segment (start 129.54 130.302) (end 133.731 126.111) (width 0.25) (layer F.Cu) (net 7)))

